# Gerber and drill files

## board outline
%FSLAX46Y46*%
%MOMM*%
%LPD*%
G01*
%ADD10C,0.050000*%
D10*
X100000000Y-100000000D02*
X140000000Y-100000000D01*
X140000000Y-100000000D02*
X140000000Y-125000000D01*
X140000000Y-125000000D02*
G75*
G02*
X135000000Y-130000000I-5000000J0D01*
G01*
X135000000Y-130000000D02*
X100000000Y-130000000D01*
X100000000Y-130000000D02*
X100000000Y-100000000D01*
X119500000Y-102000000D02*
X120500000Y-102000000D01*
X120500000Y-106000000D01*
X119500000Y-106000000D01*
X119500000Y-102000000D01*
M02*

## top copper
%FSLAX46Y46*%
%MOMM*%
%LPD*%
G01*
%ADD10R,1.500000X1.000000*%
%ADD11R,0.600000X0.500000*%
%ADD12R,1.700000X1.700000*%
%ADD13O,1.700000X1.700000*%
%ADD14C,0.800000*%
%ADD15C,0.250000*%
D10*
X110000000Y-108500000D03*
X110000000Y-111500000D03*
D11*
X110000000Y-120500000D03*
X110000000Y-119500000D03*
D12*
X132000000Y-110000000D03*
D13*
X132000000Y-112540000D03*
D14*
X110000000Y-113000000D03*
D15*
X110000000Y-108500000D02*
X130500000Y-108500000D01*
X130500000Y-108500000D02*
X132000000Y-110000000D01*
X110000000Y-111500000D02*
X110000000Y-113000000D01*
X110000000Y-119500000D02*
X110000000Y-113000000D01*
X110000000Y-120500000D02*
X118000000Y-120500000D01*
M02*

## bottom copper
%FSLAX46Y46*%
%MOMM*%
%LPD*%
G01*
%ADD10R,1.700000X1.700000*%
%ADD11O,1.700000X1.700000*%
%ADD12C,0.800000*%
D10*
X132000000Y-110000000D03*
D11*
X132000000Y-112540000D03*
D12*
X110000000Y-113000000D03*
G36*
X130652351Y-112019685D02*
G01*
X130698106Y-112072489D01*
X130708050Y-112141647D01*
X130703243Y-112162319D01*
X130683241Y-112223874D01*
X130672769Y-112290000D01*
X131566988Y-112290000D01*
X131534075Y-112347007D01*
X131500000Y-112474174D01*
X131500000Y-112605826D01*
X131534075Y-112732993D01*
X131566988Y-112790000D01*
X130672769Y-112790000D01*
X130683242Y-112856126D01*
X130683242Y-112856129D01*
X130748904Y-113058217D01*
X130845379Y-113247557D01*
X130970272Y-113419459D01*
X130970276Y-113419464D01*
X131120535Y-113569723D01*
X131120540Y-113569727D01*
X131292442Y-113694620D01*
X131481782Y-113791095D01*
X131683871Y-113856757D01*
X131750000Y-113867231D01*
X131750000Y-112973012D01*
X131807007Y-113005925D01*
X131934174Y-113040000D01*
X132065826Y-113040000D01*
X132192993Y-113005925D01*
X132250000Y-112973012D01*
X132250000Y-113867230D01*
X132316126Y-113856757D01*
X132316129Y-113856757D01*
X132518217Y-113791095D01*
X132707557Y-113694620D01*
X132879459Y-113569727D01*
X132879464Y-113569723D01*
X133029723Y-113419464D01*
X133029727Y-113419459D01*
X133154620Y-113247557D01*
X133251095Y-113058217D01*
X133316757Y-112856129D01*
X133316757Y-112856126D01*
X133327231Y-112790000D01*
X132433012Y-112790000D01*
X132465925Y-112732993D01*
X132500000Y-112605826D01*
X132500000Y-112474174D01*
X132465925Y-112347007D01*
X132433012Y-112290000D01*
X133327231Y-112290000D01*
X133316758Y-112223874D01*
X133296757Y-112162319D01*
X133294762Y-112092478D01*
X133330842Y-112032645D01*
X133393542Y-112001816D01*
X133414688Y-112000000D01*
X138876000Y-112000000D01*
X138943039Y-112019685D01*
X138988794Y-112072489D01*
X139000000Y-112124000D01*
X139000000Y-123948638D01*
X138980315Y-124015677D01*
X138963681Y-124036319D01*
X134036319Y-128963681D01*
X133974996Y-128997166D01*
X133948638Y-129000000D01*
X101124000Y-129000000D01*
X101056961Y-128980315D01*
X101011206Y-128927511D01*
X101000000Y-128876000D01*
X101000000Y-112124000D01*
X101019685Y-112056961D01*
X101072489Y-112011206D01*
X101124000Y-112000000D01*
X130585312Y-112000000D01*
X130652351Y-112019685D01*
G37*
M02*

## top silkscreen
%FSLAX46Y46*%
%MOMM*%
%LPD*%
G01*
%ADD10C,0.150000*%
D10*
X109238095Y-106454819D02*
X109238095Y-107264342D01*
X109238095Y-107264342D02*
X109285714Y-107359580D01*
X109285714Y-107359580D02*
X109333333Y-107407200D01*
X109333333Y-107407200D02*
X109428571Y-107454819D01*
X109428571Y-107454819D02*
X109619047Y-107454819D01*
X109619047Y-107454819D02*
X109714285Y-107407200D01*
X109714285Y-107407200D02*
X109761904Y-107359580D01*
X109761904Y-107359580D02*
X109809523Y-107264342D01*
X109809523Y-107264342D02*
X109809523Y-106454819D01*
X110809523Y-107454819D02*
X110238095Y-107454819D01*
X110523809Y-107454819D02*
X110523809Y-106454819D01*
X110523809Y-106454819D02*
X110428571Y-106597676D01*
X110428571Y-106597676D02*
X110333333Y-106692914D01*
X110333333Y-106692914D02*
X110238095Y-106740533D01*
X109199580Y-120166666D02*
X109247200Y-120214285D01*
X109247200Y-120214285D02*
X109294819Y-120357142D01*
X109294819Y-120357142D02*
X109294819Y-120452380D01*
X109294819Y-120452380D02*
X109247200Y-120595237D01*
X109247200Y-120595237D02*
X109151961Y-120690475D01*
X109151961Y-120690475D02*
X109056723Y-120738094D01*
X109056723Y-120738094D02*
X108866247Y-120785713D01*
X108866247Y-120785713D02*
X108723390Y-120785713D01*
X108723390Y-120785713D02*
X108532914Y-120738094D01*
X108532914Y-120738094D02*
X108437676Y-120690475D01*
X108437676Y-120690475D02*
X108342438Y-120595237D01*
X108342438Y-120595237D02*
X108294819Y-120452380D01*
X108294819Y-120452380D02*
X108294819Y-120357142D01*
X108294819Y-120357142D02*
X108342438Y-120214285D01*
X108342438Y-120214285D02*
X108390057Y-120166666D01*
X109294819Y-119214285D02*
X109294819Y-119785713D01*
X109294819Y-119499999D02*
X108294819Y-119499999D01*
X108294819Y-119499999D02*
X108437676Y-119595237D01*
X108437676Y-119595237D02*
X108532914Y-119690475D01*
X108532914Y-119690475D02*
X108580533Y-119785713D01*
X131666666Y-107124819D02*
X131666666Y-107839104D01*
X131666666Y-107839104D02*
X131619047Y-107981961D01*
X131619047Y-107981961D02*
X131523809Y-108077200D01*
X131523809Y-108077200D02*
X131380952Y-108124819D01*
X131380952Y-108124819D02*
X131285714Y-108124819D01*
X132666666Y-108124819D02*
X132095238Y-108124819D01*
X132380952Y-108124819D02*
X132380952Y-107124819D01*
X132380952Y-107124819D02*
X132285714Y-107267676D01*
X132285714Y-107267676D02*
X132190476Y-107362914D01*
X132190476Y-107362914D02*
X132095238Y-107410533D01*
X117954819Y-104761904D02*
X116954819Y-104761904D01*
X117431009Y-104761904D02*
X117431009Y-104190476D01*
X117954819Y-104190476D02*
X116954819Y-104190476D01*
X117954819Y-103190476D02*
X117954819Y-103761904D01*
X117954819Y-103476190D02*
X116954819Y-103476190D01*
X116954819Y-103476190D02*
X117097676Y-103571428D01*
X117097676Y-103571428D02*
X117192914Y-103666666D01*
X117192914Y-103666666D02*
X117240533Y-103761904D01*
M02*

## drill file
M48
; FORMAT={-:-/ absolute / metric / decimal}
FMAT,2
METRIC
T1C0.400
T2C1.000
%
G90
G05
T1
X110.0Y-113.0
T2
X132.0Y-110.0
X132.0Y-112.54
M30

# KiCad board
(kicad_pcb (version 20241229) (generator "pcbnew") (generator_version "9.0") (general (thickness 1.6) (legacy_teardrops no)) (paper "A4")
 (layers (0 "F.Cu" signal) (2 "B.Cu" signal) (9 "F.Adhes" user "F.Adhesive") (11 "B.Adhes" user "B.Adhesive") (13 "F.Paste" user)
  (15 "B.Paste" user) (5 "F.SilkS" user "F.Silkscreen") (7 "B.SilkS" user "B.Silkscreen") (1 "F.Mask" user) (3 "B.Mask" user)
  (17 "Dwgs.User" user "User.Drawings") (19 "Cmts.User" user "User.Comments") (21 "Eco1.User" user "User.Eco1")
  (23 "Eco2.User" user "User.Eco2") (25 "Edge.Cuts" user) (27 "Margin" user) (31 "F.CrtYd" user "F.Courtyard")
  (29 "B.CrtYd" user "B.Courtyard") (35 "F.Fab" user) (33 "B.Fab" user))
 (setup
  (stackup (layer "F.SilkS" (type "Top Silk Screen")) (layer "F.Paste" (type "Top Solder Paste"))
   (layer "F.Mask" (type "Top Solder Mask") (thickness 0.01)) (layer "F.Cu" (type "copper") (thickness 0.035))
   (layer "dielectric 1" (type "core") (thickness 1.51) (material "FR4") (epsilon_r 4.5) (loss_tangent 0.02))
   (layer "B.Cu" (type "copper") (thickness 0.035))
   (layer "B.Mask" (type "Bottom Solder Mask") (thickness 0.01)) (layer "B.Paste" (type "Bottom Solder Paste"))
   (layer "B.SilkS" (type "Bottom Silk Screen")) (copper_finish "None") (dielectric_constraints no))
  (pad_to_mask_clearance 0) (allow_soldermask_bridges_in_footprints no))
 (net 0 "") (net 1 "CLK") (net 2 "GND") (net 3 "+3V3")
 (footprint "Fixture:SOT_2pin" (layer "F.Cu") (at 110 110)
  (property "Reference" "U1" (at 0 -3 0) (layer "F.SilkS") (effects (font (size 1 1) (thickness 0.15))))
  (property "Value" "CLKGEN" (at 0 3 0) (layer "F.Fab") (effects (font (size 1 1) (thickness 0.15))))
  (pad "1" smd rect (at 0 -1.5) (size 1.5 1) (layers "F.Cu" "F.Paste" "F.Mask") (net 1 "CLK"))
  (pad "2" smd rect (at 0 1.5) (size 1.5 1) (layers "F.Cu" "F.Paste" "F.Mask") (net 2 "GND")))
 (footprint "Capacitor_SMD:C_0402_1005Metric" (layer "F.Cu") (at 110 120 90)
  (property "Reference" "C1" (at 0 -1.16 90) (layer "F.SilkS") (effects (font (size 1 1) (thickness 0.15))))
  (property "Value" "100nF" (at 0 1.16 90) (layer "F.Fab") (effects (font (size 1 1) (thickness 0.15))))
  (pad "1" smd rect (at -0.5 0 90) (size 0.5 0.6) (layers "F.Cu" "F.Paste" "F.Mask") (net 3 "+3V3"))
  (pad "2" smd rect (at 0.5 0 90) (size 0.5 0.6) (layers "F.Cu" "F.Paste" "F.Mask") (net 2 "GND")))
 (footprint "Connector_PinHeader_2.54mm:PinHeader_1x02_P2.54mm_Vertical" (layer "F.Cu") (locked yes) (at 132 110)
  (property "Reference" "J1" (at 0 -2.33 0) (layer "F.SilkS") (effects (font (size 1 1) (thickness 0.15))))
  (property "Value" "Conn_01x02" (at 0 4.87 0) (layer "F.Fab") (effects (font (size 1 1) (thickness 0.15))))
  (pad "1" thru_hole rect (at 0 0) (size 1.7 1.7) (drill 1) (layers "*.Cu" "*.Mask") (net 1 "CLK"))
  (pad "2" thru_hole oval (at 0 2.54) (size 1.7 1.7) (drill 1) (layers "*.Cu" "*.Mask") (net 2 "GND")))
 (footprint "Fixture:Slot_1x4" (layer "F.Cu") (at 120 104 90)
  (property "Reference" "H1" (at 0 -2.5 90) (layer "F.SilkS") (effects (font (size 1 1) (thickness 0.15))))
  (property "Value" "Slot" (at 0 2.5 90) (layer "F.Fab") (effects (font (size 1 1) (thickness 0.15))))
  (fp_rect (start -2 -0.5) (end 2 0.5) (stroke (width 0.05) (type default)) (fill no) (layer "Edge.Cuts")))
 (gr_line (start 100 100) (end 140 100) (stroke (width 0.05) (type default)) (layer "Edge.Cuts"))
 (gr_line (start 140 100) (end 140 125) (stroke (width 0.05) (type default)) (layer "Edge.Cuts"))
 (gr_arc (start 140 125) (mid 138.535534 128.535534) (end 135 130) (stroke (width 0.05) (type default)) (layer "Edge.Cuts"))
 (gr_line (start 135 130) (end 100 130) (stroke (width 0.05) (type default)) (layer "Edge.Cuts"))
 (gr_line (start 100 130) (end 100 100) (stroke (width 0.05) (type default)) (layer "Edge.Cuts"))
 (segment (start 110 108.5) (end 130.5 108.5) (width 0.25) (layer "F.Cu") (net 1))
 (segment (start 130.5 108.5) (end 132 110) (width 0.25) (layer "F.Cu") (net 1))
 (segment (start 110 111.5) (end 110 113) (width 0.25) (layer "F.Cu") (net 2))
 (segment (start 110 119.5) (end 110 113) (width 0.25) (layer "F.Cu") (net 2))
 (segment (start 110 120.5) (end 118 120.5) (width 0.25) (layer "F.Cu") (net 3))
 (via (at 110 113) (size 0.8) (drill 0.4) (layers "F.Cu" "B.Cu") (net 2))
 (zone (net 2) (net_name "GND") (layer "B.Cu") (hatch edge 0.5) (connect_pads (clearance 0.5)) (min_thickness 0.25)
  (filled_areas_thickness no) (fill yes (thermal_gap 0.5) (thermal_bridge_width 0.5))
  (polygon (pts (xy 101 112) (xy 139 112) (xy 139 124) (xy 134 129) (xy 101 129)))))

